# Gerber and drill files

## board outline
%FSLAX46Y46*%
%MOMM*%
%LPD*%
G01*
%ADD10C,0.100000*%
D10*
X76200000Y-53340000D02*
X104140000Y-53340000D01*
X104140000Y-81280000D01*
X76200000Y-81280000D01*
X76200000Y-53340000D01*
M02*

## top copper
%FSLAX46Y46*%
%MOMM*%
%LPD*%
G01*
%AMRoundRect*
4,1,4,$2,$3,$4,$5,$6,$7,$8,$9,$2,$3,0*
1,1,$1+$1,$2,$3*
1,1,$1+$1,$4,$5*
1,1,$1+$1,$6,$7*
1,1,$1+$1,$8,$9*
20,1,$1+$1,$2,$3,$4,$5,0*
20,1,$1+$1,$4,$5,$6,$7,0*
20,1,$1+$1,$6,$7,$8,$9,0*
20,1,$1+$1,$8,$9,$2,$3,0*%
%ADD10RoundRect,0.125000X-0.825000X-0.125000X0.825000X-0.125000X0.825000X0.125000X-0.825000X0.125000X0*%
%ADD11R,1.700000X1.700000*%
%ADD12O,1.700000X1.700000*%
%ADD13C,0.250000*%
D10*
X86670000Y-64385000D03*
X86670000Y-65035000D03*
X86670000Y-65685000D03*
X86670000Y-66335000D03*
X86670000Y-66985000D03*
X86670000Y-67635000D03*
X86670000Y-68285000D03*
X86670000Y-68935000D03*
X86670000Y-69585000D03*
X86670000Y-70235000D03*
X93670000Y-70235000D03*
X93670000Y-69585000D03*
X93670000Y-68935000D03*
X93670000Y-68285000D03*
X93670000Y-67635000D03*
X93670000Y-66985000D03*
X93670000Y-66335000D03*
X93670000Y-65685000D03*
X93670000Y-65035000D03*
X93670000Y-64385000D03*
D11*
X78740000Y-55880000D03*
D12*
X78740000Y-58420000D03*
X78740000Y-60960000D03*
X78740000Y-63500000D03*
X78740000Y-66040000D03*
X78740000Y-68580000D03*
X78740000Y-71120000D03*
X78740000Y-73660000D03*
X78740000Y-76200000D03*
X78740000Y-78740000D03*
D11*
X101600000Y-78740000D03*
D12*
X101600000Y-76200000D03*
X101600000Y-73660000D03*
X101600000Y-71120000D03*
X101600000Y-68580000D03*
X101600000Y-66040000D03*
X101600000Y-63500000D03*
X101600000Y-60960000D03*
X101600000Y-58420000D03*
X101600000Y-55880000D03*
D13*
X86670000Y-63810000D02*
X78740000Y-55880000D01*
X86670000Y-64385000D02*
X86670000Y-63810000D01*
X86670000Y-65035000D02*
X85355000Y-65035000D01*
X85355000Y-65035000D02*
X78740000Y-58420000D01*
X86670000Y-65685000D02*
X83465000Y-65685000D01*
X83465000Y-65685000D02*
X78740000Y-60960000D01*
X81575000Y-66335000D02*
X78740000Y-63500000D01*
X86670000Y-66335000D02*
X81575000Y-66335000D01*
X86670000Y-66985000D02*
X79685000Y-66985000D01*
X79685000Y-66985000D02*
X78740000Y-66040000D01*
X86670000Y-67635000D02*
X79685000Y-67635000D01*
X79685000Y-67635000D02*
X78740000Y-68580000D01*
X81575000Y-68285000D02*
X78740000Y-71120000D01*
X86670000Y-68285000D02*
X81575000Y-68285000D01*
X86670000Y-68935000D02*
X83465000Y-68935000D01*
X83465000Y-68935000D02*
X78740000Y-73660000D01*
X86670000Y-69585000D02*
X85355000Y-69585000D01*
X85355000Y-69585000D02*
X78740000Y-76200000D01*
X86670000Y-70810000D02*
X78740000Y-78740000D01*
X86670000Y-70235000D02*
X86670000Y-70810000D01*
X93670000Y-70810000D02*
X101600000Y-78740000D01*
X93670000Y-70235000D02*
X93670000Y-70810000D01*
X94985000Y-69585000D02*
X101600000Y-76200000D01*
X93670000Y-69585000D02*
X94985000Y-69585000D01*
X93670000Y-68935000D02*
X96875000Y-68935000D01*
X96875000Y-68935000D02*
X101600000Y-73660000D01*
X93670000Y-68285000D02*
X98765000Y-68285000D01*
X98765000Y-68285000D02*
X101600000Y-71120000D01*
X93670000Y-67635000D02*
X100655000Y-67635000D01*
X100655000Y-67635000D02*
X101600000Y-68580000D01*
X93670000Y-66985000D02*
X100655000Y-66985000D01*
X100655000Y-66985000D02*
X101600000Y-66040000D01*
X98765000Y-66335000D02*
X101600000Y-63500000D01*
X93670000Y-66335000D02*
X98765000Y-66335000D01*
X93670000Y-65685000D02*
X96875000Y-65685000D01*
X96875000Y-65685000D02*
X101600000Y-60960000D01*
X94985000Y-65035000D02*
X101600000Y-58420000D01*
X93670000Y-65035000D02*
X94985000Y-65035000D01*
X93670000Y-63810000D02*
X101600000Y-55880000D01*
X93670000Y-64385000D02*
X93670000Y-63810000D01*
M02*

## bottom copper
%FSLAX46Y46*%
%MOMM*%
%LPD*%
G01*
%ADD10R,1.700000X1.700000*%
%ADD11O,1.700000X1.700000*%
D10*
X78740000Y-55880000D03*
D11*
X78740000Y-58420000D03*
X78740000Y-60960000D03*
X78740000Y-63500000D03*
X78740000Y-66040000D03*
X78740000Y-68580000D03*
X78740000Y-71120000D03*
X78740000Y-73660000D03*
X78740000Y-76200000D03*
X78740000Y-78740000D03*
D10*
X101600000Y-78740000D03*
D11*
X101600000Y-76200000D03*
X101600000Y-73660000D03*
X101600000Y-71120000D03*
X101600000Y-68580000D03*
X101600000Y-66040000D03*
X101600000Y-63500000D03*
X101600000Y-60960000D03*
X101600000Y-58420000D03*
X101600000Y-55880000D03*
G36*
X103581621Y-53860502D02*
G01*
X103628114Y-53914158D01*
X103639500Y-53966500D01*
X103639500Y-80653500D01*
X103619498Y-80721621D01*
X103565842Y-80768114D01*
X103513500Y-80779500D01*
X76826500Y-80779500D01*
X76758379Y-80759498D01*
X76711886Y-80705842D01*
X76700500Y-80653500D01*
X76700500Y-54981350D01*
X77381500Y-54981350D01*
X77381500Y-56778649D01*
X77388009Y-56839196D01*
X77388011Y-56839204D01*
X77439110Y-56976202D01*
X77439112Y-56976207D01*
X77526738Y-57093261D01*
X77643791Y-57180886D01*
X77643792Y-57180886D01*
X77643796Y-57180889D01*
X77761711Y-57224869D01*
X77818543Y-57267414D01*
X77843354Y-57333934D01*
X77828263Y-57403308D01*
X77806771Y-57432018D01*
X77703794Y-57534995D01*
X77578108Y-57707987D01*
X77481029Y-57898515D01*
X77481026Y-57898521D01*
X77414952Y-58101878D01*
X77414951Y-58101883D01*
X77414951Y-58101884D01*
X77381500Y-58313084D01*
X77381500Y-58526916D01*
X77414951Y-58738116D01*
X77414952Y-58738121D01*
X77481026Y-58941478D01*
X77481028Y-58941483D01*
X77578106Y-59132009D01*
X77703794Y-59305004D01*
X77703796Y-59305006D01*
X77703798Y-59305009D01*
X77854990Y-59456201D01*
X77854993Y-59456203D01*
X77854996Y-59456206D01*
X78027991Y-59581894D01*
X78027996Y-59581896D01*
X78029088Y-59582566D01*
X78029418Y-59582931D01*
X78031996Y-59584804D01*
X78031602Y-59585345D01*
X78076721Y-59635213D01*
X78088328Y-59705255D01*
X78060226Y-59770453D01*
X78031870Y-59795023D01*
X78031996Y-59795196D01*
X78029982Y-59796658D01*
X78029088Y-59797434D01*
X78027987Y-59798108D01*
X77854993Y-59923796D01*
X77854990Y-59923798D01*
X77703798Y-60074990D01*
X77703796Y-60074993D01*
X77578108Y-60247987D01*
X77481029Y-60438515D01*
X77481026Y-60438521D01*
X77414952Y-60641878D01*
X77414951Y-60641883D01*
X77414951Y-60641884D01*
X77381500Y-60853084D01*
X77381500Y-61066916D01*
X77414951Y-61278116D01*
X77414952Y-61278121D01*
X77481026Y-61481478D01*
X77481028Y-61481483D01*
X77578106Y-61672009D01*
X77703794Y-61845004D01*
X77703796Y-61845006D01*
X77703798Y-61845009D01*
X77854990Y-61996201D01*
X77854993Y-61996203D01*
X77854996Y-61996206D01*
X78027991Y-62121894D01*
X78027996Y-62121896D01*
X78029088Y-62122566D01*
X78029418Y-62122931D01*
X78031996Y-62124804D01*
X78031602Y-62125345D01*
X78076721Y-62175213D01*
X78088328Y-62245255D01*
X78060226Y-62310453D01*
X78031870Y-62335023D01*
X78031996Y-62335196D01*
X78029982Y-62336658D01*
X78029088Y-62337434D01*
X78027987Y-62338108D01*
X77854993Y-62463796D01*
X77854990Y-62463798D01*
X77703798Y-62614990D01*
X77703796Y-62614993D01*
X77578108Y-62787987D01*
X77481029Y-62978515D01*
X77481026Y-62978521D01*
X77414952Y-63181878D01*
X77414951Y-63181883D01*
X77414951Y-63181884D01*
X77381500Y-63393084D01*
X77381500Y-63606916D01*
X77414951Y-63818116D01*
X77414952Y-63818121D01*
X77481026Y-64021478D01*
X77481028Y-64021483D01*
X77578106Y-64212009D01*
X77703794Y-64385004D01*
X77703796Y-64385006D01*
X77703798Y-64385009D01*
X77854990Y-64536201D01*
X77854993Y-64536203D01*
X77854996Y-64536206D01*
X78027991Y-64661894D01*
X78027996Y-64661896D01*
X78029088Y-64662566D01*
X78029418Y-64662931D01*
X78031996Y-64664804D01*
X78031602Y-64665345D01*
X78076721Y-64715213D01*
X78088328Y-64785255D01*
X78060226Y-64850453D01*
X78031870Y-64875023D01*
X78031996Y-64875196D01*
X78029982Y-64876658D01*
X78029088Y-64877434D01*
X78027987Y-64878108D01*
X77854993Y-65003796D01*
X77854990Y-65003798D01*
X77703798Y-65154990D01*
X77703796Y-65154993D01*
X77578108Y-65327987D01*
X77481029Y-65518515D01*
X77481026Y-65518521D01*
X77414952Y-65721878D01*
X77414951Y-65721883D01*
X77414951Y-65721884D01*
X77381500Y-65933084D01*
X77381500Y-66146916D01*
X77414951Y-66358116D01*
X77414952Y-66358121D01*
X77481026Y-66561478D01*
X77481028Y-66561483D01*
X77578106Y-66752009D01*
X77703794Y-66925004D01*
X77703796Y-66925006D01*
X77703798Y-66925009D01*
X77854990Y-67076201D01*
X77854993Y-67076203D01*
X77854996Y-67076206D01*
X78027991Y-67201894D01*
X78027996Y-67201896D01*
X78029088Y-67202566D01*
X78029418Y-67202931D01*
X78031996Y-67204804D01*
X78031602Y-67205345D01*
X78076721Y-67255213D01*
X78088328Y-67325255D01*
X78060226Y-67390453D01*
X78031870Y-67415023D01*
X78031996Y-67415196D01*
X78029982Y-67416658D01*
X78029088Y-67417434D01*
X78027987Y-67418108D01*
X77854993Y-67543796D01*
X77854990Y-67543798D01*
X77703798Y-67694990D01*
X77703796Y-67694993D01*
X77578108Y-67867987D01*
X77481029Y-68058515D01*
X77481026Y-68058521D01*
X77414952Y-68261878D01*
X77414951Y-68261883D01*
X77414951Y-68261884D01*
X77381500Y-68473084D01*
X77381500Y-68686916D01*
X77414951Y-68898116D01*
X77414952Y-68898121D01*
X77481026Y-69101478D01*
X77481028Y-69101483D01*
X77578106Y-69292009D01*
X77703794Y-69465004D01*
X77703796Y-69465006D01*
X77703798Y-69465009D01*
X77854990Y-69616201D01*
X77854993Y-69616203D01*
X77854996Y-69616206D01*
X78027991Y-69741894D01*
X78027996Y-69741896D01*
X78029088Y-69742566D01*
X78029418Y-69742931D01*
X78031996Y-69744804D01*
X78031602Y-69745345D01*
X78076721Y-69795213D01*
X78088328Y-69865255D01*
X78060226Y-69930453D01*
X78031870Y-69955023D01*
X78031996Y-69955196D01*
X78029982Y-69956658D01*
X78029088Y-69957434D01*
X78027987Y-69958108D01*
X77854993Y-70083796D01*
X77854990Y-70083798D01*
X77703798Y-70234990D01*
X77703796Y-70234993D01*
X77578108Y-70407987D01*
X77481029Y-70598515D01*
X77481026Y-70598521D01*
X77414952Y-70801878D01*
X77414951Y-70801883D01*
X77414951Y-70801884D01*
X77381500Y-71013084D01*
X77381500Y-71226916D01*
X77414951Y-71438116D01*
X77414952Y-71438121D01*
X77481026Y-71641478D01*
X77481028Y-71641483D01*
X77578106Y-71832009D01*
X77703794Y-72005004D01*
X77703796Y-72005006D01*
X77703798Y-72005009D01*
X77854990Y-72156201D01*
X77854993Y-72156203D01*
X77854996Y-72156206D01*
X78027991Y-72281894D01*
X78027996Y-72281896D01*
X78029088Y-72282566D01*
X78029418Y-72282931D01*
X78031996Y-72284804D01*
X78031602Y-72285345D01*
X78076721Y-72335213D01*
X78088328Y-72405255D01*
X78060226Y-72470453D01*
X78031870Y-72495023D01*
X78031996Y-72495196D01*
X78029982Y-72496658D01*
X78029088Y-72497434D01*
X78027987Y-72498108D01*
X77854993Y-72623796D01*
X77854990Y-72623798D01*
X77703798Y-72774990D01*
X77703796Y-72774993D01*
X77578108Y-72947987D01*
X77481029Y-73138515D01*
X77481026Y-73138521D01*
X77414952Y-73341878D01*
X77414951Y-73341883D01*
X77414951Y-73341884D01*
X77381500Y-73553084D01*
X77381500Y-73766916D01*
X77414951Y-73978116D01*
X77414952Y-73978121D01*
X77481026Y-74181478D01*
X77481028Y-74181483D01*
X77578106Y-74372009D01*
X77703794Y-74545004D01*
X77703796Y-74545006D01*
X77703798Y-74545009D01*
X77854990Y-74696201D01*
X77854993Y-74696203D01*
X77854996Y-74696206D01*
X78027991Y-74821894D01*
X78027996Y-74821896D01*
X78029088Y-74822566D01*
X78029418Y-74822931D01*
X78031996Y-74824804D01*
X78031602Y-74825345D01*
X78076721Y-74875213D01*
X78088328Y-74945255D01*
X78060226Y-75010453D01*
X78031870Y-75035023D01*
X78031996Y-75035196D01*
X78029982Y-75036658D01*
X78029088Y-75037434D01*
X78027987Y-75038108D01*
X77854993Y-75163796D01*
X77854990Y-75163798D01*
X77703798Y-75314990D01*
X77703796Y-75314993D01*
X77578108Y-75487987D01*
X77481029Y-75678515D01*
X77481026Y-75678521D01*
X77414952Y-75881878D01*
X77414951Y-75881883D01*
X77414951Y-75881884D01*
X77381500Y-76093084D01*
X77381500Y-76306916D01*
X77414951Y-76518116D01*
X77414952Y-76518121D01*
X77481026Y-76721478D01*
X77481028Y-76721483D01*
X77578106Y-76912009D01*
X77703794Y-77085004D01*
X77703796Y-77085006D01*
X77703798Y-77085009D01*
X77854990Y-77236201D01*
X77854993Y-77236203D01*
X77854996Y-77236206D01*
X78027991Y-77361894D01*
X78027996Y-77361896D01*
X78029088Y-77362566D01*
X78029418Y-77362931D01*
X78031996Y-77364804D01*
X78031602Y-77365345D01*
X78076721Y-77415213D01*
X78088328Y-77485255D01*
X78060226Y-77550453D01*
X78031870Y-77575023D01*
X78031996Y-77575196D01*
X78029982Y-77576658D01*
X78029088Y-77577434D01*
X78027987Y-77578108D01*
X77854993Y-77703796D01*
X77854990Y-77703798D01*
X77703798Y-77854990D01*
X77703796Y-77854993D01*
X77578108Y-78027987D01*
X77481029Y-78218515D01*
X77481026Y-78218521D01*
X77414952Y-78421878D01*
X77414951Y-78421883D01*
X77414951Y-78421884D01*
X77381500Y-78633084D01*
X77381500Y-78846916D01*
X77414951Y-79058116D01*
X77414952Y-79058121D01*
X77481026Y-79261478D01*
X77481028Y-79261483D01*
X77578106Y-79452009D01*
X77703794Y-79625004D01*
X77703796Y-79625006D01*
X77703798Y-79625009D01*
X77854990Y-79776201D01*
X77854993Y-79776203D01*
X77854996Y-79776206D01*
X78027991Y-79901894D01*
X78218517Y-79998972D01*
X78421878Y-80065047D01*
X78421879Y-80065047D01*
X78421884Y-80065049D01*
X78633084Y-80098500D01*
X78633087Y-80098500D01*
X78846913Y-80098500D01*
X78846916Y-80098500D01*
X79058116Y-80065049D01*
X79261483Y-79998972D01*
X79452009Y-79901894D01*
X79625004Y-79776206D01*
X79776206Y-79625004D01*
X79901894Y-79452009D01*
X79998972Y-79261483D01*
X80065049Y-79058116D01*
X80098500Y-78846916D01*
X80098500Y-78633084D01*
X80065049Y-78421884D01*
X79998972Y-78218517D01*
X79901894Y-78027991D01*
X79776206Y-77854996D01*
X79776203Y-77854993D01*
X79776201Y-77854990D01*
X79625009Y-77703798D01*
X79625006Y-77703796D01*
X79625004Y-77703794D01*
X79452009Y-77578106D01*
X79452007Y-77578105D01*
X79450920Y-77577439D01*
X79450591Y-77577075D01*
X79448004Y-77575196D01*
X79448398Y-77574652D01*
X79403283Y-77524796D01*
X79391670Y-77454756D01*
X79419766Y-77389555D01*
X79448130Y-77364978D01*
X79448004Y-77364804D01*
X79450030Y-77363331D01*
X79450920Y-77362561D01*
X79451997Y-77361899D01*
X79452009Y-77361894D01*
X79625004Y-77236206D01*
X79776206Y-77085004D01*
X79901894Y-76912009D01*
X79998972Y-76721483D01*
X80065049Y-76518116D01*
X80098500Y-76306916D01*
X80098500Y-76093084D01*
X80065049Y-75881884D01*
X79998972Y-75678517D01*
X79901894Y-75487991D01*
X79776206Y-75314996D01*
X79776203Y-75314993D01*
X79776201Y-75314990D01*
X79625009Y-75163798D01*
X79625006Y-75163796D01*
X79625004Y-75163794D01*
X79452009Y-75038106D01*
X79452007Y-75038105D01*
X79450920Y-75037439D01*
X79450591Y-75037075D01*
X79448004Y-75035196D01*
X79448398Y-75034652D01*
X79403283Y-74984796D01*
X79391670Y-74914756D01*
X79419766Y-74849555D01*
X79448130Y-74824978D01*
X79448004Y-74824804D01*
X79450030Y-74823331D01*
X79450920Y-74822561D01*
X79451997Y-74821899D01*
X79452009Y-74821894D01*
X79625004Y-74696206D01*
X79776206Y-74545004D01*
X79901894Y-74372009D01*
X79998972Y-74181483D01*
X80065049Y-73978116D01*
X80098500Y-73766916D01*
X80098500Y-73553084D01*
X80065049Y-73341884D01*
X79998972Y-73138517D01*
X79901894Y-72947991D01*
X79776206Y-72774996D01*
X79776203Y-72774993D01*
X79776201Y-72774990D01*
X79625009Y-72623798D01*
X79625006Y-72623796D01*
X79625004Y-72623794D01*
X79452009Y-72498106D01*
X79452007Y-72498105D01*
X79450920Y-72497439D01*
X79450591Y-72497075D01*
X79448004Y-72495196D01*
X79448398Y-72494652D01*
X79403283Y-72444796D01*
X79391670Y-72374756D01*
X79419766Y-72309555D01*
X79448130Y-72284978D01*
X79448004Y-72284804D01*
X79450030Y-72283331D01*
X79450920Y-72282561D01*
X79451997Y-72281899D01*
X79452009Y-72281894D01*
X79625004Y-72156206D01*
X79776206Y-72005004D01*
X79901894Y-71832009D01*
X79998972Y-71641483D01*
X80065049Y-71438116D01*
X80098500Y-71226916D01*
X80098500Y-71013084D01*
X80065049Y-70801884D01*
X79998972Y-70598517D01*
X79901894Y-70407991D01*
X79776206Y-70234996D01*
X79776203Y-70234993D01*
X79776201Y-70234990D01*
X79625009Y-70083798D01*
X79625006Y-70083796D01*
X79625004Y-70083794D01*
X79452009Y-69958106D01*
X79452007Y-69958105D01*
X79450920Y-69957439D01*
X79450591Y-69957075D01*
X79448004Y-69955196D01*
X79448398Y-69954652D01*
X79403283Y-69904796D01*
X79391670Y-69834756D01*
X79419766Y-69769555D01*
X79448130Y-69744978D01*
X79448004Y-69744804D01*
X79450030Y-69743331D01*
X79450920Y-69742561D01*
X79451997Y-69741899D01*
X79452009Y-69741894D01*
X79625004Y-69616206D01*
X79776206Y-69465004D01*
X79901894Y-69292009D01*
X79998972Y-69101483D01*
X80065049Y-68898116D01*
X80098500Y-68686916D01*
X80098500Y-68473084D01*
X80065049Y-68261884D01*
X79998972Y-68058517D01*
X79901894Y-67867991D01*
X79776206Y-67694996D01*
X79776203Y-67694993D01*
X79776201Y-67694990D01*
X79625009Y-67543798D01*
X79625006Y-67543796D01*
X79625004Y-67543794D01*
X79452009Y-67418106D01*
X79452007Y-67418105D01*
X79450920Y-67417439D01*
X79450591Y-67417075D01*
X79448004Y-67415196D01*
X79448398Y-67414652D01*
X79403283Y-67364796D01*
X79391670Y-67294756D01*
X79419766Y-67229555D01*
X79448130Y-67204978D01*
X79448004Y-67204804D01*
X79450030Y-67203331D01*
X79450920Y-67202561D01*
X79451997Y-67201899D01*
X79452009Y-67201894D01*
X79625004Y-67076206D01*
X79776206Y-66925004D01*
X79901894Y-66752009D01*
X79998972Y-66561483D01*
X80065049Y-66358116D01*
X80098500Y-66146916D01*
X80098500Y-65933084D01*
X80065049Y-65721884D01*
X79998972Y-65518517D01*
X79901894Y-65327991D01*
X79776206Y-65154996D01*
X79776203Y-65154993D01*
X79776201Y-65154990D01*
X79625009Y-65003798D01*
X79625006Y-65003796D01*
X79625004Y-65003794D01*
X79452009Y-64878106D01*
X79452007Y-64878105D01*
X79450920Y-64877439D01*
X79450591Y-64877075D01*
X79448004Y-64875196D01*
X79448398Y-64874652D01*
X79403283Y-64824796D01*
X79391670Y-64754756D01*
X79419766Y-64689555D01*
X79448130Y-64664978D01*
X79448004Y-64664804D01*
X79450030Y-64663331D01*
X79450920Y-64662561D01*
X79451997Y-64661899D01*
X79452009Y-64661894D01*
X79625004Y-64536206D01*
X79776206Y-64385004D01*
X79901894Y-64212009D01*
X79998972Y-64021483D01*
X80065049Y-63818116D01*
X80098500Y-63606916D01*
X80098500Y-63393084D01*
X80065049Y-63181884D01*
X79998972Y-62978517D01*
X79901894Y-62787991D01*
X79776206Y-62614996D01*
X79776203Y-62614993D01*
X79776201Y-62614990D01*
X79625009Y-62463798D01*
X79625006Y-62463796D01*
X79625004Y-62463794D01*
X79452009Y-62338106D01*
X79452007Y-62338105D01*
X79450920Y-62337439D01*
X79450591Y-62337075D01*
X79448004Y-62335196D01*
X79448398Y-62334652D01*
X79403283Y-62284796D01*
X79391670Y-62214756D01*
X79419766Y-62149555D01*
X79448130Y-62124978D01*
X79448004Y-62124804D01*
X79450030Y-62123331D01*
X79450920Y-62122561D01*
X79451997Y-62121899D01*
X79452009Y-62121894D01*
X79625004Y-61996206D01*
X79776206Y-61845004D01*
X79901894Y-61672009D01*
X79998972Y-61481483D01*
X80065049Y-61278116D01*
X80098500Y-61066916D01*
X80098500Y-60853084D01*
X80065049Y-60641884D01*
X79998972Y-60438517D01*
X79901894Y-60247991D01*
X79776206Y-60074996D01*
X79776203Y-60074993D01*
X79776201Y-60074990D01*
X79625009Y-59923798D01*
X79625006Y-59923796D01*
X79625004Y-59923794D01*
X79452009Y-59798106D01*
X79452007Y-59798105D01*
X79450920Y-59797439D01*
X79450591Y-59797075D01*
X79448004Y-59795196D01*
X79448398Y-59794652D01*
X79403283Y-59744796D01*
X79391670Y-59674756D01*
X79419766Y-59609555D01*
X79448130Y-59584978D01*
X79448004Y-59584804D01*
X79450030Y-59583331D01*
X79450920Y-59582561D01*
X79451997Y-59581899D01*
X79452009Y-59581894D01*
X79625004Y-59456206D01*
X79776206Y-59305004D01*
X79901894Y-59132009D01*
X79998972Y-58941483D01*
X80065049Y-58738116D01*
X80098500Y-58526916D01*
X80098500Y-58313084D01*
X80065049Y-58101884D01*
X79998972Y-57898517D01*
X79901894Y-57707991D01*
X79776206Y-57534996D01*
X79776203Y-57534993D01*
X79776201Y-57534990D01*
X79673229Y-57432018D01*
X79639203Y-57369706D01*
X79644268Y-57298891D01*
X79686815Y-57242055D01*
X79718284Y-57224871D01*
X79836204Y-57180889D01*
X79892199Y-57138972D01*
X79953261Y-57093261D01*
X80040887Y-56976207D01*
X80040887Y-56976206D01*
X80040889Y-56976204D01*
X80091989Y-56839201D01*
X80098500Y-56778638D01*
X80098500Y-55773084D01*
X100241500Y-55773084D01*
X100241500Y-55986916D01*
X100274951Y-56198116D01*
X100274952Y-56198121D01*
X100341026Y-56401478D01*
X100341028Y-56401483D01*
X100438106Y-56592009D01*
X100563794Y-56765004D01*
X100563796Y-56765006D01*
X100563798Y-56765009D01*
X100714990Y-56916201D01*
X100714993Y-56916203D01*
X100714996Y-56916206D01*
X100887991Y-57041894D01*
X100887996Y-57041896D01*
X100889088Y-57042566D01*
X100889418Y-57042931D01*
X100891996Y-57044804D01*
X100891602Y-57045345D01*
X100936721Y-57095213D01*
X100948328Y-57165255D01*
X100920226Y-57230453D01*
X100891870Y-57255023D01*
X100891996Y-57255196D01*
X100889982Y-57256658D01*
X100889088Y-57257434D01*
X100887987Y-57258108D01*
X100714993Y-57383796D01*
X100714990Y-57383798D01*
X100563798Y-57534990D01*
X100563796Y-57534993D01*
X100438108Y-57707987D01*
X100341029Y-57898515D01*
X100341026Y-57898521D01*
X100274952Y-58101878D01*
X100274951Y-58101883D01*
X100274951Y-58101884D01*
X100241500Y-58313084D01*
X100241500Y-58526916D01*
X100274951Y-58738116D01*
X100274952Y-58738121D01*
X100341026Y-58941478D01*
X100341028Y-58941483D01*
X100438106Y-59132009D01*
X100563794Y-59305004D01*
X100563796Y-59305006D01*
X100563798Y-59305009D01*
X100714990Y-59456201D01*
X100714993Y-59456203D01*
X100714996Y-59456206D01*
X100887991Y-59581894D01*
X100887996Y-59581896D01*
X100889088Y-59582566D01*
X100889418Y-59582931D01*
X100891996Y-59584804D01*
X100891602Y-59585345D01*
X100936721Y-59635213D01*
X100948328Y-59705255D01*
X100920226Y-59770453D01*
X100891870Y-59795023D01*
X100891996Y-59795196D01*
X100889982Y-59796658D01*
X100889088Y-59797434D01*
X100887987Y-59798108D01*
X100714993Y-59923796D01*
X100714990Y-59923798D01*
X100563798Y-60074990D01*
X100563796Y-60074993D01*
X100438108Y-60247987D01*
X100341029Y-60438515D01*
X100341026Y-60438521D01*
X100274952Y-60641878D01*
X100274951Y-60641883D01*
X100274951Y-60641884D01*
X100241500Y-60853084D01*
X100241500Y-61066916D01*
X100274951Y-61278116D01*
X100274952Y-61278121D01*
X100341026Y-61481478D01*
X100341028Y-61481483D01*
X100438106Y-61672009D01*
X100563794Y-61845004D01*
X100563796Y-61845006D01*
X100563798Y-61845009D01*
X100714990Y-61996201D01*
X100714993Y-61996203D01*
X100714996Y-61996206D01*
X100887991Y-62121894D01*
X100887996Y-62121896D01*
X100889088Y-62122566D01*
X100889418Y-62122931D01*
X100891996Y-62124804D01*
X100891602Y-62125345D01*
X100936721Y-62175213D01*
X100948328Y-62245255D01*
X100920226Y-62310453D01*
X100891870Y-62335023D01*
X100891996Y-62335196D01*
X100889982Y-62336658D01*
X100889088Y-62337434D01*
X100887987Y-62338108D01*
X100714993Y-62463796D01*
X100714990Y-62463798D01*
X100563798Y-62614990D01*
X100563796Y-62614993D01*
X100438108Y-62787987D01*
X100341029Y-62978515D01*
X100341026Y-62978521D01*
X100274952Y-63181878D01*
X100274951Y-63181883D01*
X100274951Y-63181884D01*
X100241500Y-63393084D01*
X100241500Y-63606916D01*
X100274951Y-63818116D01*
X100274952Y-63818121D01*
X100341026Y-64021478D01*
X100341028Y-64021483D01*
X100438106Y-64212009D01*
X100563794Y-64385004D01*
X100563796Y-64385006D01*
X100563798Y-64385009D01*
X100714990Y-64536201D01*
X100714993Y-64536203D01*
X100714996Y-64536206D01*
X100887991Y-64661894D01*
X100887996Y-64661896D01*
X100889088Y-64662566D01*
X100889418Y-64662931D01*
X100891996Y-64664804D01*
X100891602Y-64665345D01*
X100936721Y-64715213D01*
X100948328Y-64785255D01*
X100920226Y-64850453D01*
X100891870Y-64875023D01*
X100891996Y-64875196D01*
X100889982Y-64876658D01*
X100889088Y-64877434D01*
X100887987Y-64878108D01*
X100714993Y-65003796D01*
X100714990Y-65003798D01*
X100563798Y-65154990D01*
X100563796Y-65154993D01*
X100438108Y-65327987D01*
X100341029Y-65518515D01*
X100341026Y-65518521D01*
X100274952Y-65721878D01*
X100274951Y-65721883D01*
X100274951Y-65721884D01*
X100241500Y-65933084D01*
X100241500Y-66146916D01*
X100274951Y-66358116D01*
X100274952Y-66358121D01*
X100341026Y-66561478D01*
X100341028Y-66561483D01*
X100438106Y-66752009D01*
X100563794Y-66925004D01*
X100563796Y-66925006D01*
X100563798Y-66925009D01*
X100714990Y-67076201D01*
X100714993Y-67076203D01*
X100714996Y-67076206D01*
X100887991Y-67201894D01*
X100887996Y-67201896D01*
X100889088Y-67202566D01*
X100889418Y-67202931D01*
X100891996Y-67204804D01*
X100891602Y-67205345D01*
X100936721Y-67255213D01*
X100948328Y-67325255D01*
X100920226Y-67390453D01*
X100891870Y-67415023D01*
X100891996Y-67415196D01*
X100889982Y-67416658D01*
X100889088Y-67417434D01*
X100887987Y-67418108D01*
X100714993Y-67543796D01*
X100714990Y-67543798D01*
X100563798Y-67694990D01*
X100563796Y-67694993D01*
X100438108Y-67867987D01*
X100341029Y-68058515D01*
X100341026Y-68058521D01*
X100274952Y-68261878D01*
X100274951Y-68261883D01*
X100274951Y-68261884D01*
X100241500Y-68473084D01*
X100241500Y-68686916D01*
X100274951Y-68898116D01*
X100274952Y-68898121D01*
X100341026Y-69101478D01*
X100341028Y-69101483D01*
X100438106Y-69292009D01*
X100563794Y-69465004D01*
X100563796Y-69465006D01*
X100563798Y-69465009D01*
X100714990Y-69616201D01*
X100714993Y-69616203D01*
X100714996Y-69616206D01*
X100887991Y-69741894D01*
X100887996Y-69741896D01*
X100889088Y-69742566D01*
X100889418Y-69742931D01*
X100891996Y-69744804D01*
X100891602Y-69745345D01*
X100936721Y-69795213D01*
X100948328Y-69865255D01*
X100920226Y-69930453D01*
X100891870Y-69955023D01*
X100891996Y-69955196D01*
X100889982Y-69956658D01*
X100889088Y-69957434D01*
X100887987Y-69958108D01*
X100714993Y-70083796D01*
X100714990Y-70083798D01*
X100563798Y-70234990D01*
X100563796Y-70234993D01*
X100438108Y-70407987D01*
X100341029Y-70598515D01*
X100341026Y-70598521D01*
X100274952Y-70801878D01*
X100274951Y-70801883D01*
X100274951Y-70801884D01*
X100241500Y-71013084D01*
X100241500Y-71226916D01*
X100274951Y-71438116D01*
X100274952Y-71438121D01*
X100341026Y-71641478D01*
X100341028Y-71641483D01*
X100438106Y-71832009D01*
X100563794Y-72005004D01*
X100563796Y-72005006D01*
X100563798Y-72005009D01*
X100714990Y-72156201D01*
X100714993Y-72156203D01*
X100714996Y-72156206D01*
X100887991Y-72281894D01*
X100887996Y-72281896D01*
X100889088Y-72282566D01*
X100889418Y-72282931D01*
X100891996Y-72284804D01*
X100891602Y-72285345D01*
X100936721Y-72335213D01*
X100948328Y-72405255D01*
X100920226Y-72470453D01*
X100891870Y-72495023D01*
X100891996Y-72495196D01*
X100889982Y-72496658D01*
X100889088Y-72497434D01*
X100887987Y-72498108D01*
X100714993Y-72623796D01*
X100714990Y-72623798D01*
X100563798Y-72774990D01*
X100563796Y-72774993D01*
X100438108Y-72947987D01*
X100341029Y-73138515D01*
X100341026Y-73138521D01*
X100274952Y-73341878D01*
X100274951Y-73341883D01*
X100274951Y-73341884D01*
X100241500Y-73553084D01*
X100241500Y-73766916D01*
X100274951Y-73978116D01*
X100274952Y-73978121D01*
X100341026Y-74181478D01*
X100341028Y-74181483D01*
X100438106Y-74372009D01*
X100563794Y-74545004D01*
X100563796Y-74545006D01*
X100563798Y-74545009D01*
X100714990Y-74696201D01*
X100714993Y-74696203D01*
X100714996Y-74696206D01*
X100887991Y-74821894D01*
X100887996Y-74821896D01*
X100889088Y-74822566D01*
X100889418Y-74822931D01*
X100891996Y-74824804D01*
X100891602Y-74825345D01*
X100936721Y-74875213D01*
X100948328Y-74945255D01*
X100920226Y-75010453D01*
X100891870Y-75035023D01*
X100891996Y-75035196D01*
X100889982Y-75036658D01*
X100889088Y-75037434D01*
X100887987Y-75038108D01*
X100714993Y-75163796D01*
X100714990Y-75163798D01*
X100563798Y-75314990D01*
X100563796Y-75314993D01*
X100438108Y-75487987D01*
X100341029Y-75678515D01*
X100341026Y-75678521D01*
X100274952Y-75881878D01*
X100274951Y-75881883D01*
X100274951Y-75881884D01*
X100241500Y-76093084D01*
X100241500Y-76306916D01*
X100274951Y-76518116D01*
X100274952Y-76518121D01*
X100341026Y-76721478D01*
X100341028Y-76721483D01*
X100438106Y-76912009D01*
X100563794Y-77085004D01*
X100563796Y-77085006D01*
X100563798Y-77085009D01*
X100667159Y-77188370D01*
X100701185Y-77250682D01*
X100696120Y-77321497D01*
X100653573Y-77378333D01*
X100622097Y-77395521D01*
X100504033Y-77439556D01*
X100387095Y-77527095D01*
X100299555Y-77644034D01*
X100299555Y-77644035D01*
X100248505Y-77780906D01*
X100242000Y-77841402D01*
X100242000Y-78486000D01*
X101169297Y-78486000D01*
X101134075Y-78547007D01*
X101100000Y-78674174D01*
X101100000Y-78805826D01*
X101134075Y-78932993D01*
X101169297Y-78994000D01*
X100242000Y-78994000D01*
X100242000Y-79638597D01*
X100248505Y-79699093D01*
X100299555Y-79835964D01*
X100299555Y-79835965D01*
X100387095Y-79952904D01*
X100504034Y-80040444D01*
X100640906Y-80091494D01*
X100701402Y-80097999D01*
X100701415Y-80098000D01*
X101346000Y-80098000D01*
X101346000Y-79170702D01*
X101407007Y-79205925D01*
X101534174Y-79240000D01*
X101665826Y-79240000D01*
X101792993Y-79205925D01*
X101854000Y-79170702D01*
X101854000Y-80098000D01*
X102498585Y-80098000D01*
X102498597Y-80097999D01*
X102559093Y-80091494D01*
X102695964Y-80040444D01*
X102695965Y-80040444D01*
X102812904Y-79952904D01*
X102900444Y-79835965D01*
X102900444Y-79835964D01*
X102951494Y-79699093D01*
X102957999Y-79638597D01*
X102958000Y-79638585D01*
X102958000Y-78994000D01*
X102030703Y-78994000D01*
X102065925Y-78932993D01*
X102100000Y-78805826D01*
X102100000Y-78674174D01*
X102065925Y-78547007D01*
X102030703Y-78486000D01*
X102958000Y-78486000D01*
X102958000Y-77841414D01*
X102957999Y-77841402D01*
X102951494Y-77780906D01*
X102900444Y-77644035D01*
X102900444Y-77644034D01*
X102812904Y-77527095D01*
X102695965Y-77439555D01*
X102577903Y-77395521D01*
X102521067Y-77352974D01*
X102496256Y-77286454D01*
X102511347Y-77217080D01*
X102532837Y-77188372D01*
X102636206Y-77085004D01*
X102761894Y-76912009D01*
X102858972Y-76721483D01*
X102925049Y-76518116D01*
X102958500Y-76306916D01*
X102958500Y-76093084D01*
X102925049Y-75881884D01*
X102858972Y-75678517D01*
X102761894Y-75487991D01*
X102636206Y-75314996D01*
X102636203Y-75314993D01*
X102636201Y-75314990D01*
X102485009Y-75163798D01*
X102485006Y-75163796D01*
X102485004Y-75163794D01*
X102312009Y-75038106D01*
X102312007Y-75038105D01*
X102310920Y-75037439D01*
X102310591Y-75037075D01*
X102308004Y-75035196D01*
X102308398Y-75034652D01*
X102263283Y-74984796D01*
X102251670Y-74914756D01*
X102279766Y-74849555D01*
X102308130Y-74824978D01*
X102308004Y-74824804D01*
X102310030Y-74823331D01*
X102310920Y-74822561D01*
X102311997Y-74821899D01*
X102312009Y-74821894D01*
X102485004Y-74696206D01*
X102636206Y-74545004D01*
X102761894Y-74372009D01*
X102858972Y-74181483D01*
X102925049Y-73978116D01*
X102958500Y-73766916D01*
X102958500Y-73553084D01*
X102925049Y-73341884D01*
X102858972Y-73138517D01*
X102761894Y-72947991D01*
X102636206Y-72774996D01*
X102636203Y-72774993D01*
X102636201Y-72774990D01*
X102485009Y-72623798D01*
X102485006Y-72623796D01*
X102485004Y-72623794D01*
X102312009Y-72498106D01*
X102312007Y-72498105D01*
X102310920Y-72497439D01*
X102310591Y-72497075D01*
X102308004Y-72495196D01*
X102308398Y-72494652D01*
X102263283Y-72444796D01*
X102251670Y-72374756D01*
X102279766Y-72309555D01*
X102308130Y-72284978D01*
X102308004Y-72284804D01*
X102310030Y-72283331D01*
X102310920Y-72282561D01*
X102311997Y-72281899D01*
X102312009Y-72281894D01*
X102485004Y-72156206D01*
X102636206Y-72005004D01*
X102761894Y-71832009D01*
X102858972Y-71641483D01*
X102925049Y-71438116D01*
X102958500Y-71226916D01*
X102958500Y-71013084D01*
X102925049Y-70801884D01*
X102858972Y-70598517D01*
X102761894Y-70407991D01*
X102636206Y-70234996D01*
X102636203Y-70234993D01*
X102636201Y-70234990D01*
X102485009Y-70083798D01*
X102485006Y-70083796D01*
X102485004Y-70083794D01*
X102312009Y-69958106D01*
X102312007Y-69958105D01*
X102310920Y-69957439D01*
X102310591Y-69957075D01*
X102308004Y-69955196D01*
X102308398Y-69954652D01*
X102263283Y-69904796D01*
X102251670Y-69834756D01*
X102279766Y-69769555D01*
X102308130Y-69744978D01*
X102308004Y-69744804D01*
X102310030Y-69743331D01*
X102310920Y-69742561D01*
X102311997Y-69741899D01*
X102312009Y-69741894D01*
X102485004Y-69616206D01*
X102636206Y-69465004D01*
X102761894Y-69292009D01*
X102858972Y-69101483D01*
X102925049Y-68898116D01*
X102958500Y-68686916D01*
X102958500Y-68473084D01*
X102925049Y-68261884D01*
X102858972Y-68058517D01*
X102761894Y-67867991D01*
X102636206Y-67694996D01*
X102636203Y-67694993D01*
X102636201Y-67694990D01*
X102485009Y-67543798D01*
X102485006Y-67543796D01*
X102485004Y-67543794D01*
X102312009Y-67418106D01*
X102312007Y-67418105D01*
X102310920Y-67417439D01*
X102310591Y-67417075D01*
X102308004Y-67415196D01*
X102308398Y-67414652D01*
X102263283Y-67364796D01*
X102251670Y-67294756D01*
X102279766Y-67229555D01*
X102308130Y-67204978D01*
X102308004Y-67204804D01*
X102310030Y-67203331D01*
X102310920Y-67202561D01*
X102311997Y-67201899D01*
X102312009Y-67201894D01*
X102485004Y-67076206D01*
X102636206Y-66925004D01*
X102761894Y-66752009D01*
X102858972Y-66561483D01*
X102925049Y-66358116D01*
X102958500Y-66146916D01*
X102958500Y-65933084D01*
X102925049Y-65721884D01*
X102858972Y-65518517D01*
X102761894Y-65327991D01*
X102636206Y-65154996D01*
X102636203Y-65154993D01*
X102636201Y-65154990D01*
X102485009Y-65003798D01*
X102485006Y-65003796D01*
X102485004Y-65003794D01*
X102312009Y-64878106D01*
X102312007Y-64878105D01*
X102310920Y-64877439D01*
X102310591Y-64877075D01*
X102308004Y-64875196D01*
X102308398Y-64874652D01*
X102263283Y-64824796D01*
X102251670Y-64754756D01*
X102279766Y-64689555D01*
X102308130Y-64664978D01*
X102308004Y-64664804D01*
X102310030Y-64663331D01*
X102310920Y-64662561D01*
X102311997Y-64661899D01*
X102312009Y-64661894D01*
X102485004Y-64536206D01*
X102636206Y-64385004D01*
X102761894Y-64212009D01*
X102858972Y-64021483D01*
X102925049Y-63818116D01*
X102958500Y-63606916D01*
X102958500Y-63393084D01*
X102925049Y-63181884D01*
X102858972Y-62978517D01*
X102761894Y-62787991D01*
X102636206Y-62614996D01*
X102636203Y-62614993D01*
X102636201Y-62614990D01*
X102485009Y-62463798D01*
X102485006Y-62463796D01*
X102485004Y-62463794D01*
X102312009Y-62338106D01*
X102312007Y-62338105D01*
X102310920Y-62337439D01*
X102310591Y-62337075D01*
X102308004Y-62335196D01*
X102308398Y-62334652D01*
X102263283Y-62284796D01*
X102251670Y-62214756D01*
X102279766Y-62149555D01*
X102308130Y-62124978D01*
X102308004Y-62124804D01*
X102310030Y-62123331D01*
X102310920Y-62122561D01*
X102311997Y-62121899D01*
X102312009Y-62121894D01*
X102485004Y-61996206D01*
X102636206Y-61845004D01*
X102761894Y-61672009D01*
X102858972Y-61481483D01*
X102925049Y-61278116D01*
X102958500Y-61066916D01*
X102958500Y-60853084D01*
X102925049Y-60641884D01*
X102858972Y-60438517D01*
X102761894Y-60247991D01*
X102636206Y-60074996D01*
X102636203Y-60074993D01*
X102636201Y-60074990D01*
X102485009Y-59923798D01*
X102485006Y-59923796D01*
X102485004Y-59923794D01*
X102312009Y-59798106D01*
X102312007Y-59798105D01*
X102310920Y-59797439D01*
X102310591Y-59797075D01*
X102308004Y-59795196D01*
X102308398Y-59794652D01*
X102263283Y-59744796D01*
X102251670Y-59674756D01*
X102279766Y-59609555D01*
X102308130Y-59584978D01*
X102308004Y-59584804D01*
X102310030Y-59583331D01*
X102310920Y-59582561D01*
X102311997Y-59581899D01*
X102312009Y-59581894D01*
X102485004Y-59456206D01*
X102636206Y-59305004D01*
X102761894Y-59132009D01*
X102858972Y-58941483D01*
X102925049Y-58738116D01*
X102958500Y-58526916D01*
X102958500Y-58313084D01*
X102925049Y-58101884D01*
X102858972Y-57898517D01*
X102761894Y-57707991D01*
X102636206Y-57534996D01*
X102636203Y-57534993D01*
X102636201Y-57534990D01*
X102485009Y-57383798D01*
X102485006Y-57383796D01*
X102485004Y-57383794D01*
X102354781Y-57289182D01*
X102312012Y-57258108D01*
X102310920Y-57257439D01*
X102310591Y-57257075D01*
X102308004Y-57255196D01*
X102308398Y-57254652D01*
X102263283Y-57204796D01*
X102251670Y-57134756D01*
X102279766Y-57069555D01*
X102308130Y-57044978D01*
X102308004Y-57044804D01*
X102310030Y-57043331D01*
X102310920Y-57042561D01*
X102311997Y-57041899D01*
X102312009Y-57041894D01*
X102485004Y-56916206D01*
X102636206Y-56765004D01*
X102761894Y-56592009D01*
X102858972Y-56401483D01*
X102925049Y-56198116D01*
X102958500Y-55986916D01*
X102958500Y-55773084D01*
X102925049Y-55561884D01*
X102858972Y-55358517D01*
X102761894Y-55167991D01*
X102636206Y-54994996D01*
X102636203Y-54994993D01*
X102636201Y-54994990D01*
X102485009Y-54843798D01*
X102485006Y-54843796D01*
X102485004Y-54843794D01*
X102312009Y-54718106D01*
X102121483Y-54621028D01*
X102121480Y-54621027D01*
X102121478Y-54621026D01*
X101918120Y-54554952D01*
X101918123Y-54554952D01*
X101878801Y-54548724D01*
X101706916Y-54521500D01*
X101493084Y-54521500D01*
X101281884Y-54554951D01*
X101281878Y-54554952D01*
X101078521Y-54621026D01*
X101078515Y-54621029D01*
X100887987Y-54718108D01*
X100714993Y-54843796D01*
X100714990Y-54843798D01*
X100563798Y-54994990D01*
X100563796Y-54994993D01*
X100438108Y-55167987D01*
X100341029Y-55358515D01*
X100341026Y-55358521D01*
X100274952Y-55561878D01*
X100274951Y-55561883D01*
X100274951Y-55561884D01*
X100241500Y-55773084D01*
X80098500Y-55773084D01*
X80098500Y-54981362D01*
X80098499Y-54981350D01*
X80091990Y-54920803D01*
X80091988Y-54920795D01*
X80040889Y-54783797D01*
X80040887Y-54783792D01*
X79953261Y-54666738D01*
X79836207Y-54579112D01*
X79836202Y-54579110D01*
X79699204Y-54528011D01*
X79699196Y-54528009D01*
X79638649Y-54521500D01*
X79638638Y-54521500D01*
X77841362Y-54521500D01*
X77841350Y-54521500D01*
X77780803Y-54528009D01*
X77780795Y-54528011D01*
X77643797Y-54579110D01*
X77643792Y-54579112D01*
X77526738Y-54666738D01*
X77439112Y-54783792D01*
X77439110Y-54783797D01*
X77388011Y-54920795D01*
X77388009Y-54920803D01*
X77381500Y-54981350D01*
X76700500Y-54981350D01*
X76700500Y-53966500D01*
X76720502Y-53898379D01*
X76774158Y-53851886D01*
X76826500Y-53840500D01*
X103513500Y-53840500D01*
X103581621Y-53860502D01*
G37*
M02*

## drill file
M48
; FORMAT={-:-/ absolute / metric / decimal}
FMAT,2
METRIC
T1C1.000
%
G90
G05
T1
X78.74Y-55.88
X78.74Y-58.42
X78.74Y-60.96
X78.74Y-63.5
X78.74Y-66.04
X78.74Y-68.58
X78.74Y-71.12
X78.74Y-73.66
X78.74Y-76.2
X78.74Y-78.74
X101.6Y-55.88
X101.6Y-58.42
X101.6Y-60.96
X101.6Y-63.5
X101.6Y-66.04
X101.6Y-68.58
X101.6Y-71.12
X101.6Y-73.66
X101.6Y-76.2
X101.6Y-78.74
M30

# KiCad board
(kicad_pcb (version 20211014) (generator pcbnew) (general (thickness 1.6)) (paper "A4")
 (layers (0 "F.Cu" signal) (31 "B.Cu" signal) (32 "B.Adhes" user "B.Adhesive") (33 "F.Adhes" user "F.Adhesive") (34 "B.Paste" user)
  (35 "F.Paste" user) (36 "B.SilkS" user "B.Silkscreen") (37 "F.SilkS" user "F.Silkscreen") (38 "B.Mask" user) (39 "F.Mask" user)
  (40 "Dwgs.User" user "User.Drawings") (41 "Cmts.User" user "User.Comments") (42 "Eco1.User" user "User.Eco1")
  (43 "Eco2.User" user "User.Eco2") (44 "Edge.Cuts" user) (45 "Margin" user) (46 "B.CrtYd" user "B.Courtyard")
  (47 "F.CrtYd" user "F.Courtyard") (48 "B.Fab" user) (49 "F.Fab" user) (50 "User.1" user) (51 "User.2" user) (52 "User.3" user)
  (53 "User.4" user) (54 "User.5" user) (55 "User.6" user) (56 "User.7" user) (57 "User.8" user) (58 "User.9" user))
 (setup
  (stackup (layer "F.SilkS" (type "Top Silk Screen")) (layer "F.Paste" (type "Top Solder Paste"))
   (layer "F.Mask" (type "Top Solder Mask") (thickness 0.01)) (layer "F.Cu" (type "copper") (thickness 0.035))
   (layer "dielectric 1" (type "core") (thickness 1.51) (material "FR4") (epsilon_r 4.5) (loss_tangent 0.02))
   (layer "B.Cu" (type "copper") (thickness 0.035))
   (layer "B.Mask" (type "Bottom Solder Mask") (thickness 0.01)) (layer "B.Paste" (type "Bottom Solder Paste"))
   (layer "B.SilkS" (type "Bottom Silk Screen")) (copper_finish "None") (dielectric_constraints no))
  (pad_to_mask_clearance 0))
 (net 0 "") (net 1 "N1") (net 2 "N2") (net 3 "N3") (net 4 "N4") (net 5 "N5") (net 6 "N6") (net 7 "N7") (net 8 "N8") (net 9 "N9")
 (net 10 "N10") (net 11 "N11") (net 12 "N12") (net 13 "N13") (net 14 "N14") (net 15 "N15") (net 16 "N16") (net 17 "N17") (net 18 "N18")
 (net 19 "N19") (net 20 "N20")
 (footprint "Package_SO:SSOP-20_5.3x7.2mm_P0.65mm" (layer "F.Cu") (at 90.17 67.31)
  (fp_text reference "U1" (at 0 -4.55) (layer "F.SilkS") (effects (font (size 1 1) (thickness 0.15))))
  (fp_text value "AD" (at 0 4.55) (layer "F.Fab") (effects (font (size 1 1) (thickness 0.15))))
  (pad "1" smd roundrect (at -3.5 -2.925) (size 1.9 0.5) (layers "F.Cu" "F.Paste" "F.Mask") (roundrect_rratio 0.25) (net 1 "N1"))
  (pad "2" smd roundrect (at -3.5 -2.275) (size 1.9 0.5) (layers "F.Cu" "F.Paste" "F.Mask") (roundrect_rratio 0.25) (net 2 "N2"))
  (pad "3" smd roundrect (at -3.5 -1.625) (size 1.9 0.5) (layers "F.Cu" "F.Paste" "F.Mask") (roundrect_rratio 0.25) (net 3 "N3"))
  (pad "4" smd roundrect (at -3.5 -0.975) (size 1.9 0.5) (layers "F.Cu" "F.Paste" "F.Mask") (roundrect_rratio 0.25) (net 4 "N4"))
  (pad "5" smd roundrect (at -3.5 -0.325) (size 1.9 0.5) (layers "F.Cu" "F.Paste" "F.Mask") (roundrect_rratio 0.25) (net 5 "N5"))
  (pad "6" smd roundrect (at -3.5 0.325) (size 1.9 0.5) (layers "F.Cu" "F.Paste" "F.Mask") (roundrect_rratio 0.25) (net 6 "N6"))
  (pad "7" smd roundrect (at -3.5 0.975) (size 1.9 0.5) (layers "F.Cu" "F.Paste" "F.Mask") (roundrect_rratio 0.25) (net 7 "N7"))
  (pad "8" smd roundrect (at -3.5 1.625) (size 1.9 0.5) (layers "F.Cu" "F.Paste" "F.Mask") (roundrect_rratio 0.25) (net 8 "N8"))
  (pad "9" smd roundrect (at -3.5 2.275) (size 1.9 0.5) (layers "F.Cu" "F.Paste" "F.Mask") (roundrect_rratio 0.25) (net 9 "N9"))
  (pad "10" smd roundrect (at -3.5 2.925) (size 1.9 0.5) (layers "F.Cu" "F.Paste" "F.Mask") (roundrect_rratio 0.25) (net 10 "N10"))
  (pad "11" smd roundrect (at 3.5 2.925) (size 1.9 0.5) (layers "F.Cu" "F.Paste" "F.Mask") (roundrect_rratio 0.25) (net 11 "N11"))
  (pad "12" smd roundrect (at 3.5 2.275) (size 1.9 0.5) (layers "F.Cu" "F.Paste" "F.Mask") (roundrect_rratio 0.25) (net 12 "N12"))
  (pad "13" smd roundrect (at 3.5 1.625) (size 1.9 0.5) (layers "F.Cu" "F.Paste" "F.Mask") (roundrect_rratio 0.25) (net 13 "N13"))
  (pad "14" smd roundrect (at 3.5 0.975) (size 1.9 0.5) (layers "F.Cu" "F.Paste" "F.Mask") (roundrect_rratio 0.25) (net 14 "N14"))
  (pad "15" smd roundrect (at 3.5 0.325) (size 1.9 0.5) (layers "F.Cu" "F.Paste" "F.Mask") (roundrect_rratio 0.25) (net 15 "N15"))
  (pad "16" smd roundrect (at 3.5 -0.325) (size 1.9 0.5) (layers "F.Cu" "F.Paste" "F.Mask") (roundrect_rratio 0.25) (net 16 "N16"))
  (pad "17" smd roundrect (at 3.5 -0.975) (size 1.9 0.5) (layers "F.Cu" "F.Paste" "F.Mask") (roundrect_rratio 0.25) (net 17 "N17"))
  (pad "18" smd roundrect (at 3.5 -1.625) (size 1.9 0.5) (layers "F.Cu" "F.Paste" "F.Mask") (roundrect_rratio 0.25) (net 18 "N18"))
  (pad "19" smd roundrect (at 3.5 -2.275) (size 1.9 0.5) (layers "F.Cu" "F.Paste" "F.Mask") (roundrect_rratio 0.25) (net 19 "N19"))
  (pad "20" smd roundrect (at 3.5 -2.925) (size 1.9 0.5) (layers "F.Cu" "F.Paste" "F.Mask") (roundrect_rratio 0.25) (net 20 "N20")))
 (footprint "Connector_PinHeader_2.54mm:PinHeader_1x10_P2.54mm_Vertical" (layer "F.Cu") (at 78.74 55.88)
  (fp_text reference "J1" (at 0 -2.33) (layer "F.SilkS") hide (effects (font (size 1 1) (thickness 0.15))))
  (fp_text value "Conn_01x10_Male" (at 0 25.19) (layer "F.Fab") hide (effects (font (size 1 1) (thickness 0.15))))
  (pad "1" thru_hole rect (at 0 0) (size 1.7 1.7) (drill 1) (layers *.Cu *.Mask) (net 1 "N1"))
  (pad "2" thru_hole oval (at 0 2.54) (size 1.7 1.7) (drill 1) (layers *.Cu *.Mask) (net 2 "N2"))
  (pad "3" thru_hole oval (at 0 5.08) (size 1.7 1.7) (drill 1) (layers *.Cu *.Mask) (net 3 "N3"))
  (pad "4" thru_hole oval (at 0 7.62) (size 1.7 1.7) (drill 1) (layers *.Cu *.Mask) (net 4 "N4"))
  (pad "5" thru_hole oval (at 0 10.16) (size 1.7 1.7) (drill 1) (layers *.Cu *.Mask) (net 5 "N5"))
  (pad "6" thru_hole oval (at 0 12.7) (size 1.7 1.7) (drill 1) (layers *.Cu *.Mask) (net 6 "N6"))
  (pad "7" thru_hole oval (at 0 15.24) (size 1.7 1.7) (drill 1) (layers *.Cu *.Mask) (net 7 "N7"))
  (pad "8" thru_hole oval (at 0 17.78) (size 1.7 1.7) (drill 1) (layers *.Cu *.Mask) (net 8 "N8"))
  (pad "9" thru_hole oval (at 0 20.32) (size 1.7 1.7) (drill 1) (layers *.Cu *.Mask) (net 9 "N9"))
  (pad "10" thru_hole oval (at 0 22.86) (size 1.7 1.7) (drill 1) (layers *.Cu *.Mask) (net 10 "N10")))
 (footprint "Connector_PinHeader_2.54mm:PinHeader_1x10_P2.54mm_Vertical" (layer "F.Cu") (at 101.6 78.74 180)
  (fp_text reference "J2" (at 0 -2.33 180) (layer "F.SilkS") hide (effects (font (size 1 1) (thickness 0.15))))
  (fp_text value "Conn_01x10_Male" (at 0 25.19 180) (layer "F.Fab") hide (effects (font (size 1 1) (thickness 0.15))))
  (pad "1" thru_hole rect (at 0 0 180) (size 1.7 1.7) (drill 1) (layers *.Cu *.Mask) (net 11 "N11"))
  (pad "2" thru_hole oval (at 0 2.54 180) (size 1.7 1.7) (drill 1) (layers *.Cu *.Mask) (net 12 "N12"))
  (pad "3" thru_hole oval (at 0 5.08 180) (size 1.7 1.7) (drill 1) (layers *.Cu *.Mask) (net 13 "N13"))
  (pad "4" thru_hole oval (at 0 7.62 180) (size 1.7 1.7) (drill 1) (layers *.Cu *.Mask) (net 14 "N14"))
  (pad "5" thru_hole oval (at 0 10.16 180) (size 1.7 1.7) (drill 1) (layers *.Cu *.Mask) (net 15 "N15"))
  (pad "6" thru_hole oval (at 0 12.7 180) (size 1.7 1.7) (drill 1) (layers *.Cu *.Mask) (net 16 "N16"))
  (pad "7" thru_hole oval (at 0 15.24 180) (size 1.7 1.7) (drill 1) (layers *.Cu *.Mask) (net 17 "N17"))
  (pad "8" thru_hole oval (at 0 17.78 180) (size 1.7 1.7) (drill 1) (layers *.Cu *.Mask) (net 18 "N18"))
  (pad "9" thru_hole oval (at 0 20.32 180) (size 1.7 1.7) (drill 1) (layers *.Cu *.Mask) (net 19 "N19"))
  (pad "10" thru_hole oval (at 0 22.86 180) (size 1.7 1.7) (drill 1) (layers *.Cu *.Mask) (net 20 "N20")))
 (gr_rect (start 104.14 53.34) (end 76.2 81.28) (layer "Edge.Cuts") (width 0.1) (fill none))
 (segment (start 86.67 63.81) (end 78.74 55.88) (width 0.25) (layer "F.Cu") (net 1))
 (segment (start 86.67 64.385) (end 86.67 63.81) (width 0.25) (layer "F.Cu") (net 1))
 (segment (start 86.67 65.035) (end 85.355 65.035) (width 0.25) (layer "F.Cu") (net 2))
 (segment (start 85.355 65.035) (end 78.74 58.42) (width 0.25) (layer "F.Cu") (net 2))
 (segment (start 86.67 65.685) (end 83.465 65.685) (width 0.25) (layer "F.Cu") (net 3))
 (segment (start 83.465 65.685) (end 78.74 60.96) (width 0.25) (layer "F.Cu") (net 3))
 (segment (start 81.575 66.335) (end 78.74 63.5) (width 0.25) (layer "F.Cu") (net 4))
 (segment (start 86.67 66.335) (end 81.575 66.335) (width 0.25) (layer "F.Cu") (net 4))
 (segment (start 86.67 66.985) (end 79.685 66.985) (width 0.25) (layer "F.Cu") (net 5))
 (segment (start 79.685 66.985) (end 78.74 66.04) (width 0.25) (layer "F.Cu") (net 5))
 (segment (start 86.67 67.635) (end 79.685 67.635) (width 0.25) (layer "F.Cu") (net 6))
 (segment (start 79.685 67.635) (end 78.74 68.58) (width 0.25) (layer "F.Cu") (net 6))
 (segment (start 81.575 68.285) (end 78.74 71.12) (width 0.25) (layer "F.Cu") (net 7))
 (segment (start 86.67 68.285) (end 81.575 68.285) (width 0.25) (layer "F.Cu") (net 7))
 (segment (start 86.67 68.935) (end 83.465 68.935) (width 0.25) (layer "F.Cu") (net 8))
 (segment (start 83.465 68.935) (end 78.74 73.66) (width 0.25) (layer "F.Cu") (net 8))
 (segment (start 86.67 69.585) (end 85.355 69.585) (width 0.25) (layer "F.Cu") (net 9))
 (segment (start 85.355 69.585) (end 78.74 76.2) (width 0.25) (layer "F.Cu") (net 9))
 (segment (start 86.67 70.81) (end 78.74 78.74) (width 0.25) (layer "F.Cu") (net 10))
 (segment (start 86.67 70.235) (end 86.67 70.81) (width 0.25) (layer "F.Cu") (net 10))
 (segment (start 93.67 70.81) (end 101.6 78.74) (width 0.25) (layer "F.Cu") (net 11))
 (segment (start 93.67 70.235) (end 93.67 70.81) (width 0.25) (layer "F.Cu") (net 11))
 (segment (start 94.985 69.585) (end 101.6 76.2) (width 0.25) (layer "F.Cu") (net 12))
 (segment (start 93.67 69.585) (end 94.985 69.585) (width 0.25) (layer "F.Cu") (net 12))
 (segment (start 93.67 68.935) (end 96.875 68.935) (width 0.25) (layer "F.Cu") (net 13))
 (segment (start 96.875 68.935) (end 101.6 73.66) (width 0.25) (layer "F.Cu") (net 13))
 (segment (start 93.67 68.285) (end 98.765 68.285) (width 0.25) (layer "F.Cu") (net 14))
 (segment (start 98.765 68.285) (end 101.6 71.12) (width 0.25) (layer "F.Cu") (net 14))
 (segment (start 93.67 67.635) (end 100.655 67.635) (width 0.25) (layer "F.Cu") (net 15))
 (segment (start 100.655 67.635) (end 101.6 68.58) (width 0.25) (layer "F.Cu") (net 15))
 (segment (start 93.67 66.985) (end 100.655 66.985) (width 0.25) (layer "F.Cu") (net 16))
 (segment (start 100.655 66.985) (end 101.6 66.04) (width 0.25) (layer "F.Cu") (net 16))
 (segment (start 98.765 66.335) (end 101.6 63.5) (width 0.25) (layer "F.Cu") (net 17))
 (segment (start 93.67 66.335) (end 98.765 66.335) (width 0.25) (layer "F.Cu") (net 17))
 (segment (start 93.67 65.685) (end 96.875 65.685) (width 0.25) (layer "F.Cu") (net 18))
 (segment (start 96.875 65.685) (end 101.6 60.96) (width 0.25) (layer "F.Cu") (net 18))
 (segment (start 94.985 65.035) (end 101.6 58.42) (width 0.25) (layer "F.Cu") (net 19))
 (segment (start 93.67 65.035) (end 94.985 65.035) (width 0.25) (layer "F.Cu") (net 19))
 (segment (start 93.67 63.81) (end 101.6 55.88) (width 0.25) (layer "F.Cu") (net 20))
 (segment (start 93.67 64.385) (end 93.67 63.81) (width 0.25) (layer "F.Cu") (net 20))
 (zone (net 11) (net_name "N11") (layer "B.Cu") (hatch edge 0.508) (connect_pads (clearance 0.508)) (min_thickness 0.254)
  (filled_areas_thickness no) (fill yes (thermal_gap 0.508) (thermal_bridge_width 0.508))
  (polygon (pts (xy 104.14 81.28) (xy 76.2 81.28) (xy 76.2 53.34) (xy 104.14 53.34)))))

